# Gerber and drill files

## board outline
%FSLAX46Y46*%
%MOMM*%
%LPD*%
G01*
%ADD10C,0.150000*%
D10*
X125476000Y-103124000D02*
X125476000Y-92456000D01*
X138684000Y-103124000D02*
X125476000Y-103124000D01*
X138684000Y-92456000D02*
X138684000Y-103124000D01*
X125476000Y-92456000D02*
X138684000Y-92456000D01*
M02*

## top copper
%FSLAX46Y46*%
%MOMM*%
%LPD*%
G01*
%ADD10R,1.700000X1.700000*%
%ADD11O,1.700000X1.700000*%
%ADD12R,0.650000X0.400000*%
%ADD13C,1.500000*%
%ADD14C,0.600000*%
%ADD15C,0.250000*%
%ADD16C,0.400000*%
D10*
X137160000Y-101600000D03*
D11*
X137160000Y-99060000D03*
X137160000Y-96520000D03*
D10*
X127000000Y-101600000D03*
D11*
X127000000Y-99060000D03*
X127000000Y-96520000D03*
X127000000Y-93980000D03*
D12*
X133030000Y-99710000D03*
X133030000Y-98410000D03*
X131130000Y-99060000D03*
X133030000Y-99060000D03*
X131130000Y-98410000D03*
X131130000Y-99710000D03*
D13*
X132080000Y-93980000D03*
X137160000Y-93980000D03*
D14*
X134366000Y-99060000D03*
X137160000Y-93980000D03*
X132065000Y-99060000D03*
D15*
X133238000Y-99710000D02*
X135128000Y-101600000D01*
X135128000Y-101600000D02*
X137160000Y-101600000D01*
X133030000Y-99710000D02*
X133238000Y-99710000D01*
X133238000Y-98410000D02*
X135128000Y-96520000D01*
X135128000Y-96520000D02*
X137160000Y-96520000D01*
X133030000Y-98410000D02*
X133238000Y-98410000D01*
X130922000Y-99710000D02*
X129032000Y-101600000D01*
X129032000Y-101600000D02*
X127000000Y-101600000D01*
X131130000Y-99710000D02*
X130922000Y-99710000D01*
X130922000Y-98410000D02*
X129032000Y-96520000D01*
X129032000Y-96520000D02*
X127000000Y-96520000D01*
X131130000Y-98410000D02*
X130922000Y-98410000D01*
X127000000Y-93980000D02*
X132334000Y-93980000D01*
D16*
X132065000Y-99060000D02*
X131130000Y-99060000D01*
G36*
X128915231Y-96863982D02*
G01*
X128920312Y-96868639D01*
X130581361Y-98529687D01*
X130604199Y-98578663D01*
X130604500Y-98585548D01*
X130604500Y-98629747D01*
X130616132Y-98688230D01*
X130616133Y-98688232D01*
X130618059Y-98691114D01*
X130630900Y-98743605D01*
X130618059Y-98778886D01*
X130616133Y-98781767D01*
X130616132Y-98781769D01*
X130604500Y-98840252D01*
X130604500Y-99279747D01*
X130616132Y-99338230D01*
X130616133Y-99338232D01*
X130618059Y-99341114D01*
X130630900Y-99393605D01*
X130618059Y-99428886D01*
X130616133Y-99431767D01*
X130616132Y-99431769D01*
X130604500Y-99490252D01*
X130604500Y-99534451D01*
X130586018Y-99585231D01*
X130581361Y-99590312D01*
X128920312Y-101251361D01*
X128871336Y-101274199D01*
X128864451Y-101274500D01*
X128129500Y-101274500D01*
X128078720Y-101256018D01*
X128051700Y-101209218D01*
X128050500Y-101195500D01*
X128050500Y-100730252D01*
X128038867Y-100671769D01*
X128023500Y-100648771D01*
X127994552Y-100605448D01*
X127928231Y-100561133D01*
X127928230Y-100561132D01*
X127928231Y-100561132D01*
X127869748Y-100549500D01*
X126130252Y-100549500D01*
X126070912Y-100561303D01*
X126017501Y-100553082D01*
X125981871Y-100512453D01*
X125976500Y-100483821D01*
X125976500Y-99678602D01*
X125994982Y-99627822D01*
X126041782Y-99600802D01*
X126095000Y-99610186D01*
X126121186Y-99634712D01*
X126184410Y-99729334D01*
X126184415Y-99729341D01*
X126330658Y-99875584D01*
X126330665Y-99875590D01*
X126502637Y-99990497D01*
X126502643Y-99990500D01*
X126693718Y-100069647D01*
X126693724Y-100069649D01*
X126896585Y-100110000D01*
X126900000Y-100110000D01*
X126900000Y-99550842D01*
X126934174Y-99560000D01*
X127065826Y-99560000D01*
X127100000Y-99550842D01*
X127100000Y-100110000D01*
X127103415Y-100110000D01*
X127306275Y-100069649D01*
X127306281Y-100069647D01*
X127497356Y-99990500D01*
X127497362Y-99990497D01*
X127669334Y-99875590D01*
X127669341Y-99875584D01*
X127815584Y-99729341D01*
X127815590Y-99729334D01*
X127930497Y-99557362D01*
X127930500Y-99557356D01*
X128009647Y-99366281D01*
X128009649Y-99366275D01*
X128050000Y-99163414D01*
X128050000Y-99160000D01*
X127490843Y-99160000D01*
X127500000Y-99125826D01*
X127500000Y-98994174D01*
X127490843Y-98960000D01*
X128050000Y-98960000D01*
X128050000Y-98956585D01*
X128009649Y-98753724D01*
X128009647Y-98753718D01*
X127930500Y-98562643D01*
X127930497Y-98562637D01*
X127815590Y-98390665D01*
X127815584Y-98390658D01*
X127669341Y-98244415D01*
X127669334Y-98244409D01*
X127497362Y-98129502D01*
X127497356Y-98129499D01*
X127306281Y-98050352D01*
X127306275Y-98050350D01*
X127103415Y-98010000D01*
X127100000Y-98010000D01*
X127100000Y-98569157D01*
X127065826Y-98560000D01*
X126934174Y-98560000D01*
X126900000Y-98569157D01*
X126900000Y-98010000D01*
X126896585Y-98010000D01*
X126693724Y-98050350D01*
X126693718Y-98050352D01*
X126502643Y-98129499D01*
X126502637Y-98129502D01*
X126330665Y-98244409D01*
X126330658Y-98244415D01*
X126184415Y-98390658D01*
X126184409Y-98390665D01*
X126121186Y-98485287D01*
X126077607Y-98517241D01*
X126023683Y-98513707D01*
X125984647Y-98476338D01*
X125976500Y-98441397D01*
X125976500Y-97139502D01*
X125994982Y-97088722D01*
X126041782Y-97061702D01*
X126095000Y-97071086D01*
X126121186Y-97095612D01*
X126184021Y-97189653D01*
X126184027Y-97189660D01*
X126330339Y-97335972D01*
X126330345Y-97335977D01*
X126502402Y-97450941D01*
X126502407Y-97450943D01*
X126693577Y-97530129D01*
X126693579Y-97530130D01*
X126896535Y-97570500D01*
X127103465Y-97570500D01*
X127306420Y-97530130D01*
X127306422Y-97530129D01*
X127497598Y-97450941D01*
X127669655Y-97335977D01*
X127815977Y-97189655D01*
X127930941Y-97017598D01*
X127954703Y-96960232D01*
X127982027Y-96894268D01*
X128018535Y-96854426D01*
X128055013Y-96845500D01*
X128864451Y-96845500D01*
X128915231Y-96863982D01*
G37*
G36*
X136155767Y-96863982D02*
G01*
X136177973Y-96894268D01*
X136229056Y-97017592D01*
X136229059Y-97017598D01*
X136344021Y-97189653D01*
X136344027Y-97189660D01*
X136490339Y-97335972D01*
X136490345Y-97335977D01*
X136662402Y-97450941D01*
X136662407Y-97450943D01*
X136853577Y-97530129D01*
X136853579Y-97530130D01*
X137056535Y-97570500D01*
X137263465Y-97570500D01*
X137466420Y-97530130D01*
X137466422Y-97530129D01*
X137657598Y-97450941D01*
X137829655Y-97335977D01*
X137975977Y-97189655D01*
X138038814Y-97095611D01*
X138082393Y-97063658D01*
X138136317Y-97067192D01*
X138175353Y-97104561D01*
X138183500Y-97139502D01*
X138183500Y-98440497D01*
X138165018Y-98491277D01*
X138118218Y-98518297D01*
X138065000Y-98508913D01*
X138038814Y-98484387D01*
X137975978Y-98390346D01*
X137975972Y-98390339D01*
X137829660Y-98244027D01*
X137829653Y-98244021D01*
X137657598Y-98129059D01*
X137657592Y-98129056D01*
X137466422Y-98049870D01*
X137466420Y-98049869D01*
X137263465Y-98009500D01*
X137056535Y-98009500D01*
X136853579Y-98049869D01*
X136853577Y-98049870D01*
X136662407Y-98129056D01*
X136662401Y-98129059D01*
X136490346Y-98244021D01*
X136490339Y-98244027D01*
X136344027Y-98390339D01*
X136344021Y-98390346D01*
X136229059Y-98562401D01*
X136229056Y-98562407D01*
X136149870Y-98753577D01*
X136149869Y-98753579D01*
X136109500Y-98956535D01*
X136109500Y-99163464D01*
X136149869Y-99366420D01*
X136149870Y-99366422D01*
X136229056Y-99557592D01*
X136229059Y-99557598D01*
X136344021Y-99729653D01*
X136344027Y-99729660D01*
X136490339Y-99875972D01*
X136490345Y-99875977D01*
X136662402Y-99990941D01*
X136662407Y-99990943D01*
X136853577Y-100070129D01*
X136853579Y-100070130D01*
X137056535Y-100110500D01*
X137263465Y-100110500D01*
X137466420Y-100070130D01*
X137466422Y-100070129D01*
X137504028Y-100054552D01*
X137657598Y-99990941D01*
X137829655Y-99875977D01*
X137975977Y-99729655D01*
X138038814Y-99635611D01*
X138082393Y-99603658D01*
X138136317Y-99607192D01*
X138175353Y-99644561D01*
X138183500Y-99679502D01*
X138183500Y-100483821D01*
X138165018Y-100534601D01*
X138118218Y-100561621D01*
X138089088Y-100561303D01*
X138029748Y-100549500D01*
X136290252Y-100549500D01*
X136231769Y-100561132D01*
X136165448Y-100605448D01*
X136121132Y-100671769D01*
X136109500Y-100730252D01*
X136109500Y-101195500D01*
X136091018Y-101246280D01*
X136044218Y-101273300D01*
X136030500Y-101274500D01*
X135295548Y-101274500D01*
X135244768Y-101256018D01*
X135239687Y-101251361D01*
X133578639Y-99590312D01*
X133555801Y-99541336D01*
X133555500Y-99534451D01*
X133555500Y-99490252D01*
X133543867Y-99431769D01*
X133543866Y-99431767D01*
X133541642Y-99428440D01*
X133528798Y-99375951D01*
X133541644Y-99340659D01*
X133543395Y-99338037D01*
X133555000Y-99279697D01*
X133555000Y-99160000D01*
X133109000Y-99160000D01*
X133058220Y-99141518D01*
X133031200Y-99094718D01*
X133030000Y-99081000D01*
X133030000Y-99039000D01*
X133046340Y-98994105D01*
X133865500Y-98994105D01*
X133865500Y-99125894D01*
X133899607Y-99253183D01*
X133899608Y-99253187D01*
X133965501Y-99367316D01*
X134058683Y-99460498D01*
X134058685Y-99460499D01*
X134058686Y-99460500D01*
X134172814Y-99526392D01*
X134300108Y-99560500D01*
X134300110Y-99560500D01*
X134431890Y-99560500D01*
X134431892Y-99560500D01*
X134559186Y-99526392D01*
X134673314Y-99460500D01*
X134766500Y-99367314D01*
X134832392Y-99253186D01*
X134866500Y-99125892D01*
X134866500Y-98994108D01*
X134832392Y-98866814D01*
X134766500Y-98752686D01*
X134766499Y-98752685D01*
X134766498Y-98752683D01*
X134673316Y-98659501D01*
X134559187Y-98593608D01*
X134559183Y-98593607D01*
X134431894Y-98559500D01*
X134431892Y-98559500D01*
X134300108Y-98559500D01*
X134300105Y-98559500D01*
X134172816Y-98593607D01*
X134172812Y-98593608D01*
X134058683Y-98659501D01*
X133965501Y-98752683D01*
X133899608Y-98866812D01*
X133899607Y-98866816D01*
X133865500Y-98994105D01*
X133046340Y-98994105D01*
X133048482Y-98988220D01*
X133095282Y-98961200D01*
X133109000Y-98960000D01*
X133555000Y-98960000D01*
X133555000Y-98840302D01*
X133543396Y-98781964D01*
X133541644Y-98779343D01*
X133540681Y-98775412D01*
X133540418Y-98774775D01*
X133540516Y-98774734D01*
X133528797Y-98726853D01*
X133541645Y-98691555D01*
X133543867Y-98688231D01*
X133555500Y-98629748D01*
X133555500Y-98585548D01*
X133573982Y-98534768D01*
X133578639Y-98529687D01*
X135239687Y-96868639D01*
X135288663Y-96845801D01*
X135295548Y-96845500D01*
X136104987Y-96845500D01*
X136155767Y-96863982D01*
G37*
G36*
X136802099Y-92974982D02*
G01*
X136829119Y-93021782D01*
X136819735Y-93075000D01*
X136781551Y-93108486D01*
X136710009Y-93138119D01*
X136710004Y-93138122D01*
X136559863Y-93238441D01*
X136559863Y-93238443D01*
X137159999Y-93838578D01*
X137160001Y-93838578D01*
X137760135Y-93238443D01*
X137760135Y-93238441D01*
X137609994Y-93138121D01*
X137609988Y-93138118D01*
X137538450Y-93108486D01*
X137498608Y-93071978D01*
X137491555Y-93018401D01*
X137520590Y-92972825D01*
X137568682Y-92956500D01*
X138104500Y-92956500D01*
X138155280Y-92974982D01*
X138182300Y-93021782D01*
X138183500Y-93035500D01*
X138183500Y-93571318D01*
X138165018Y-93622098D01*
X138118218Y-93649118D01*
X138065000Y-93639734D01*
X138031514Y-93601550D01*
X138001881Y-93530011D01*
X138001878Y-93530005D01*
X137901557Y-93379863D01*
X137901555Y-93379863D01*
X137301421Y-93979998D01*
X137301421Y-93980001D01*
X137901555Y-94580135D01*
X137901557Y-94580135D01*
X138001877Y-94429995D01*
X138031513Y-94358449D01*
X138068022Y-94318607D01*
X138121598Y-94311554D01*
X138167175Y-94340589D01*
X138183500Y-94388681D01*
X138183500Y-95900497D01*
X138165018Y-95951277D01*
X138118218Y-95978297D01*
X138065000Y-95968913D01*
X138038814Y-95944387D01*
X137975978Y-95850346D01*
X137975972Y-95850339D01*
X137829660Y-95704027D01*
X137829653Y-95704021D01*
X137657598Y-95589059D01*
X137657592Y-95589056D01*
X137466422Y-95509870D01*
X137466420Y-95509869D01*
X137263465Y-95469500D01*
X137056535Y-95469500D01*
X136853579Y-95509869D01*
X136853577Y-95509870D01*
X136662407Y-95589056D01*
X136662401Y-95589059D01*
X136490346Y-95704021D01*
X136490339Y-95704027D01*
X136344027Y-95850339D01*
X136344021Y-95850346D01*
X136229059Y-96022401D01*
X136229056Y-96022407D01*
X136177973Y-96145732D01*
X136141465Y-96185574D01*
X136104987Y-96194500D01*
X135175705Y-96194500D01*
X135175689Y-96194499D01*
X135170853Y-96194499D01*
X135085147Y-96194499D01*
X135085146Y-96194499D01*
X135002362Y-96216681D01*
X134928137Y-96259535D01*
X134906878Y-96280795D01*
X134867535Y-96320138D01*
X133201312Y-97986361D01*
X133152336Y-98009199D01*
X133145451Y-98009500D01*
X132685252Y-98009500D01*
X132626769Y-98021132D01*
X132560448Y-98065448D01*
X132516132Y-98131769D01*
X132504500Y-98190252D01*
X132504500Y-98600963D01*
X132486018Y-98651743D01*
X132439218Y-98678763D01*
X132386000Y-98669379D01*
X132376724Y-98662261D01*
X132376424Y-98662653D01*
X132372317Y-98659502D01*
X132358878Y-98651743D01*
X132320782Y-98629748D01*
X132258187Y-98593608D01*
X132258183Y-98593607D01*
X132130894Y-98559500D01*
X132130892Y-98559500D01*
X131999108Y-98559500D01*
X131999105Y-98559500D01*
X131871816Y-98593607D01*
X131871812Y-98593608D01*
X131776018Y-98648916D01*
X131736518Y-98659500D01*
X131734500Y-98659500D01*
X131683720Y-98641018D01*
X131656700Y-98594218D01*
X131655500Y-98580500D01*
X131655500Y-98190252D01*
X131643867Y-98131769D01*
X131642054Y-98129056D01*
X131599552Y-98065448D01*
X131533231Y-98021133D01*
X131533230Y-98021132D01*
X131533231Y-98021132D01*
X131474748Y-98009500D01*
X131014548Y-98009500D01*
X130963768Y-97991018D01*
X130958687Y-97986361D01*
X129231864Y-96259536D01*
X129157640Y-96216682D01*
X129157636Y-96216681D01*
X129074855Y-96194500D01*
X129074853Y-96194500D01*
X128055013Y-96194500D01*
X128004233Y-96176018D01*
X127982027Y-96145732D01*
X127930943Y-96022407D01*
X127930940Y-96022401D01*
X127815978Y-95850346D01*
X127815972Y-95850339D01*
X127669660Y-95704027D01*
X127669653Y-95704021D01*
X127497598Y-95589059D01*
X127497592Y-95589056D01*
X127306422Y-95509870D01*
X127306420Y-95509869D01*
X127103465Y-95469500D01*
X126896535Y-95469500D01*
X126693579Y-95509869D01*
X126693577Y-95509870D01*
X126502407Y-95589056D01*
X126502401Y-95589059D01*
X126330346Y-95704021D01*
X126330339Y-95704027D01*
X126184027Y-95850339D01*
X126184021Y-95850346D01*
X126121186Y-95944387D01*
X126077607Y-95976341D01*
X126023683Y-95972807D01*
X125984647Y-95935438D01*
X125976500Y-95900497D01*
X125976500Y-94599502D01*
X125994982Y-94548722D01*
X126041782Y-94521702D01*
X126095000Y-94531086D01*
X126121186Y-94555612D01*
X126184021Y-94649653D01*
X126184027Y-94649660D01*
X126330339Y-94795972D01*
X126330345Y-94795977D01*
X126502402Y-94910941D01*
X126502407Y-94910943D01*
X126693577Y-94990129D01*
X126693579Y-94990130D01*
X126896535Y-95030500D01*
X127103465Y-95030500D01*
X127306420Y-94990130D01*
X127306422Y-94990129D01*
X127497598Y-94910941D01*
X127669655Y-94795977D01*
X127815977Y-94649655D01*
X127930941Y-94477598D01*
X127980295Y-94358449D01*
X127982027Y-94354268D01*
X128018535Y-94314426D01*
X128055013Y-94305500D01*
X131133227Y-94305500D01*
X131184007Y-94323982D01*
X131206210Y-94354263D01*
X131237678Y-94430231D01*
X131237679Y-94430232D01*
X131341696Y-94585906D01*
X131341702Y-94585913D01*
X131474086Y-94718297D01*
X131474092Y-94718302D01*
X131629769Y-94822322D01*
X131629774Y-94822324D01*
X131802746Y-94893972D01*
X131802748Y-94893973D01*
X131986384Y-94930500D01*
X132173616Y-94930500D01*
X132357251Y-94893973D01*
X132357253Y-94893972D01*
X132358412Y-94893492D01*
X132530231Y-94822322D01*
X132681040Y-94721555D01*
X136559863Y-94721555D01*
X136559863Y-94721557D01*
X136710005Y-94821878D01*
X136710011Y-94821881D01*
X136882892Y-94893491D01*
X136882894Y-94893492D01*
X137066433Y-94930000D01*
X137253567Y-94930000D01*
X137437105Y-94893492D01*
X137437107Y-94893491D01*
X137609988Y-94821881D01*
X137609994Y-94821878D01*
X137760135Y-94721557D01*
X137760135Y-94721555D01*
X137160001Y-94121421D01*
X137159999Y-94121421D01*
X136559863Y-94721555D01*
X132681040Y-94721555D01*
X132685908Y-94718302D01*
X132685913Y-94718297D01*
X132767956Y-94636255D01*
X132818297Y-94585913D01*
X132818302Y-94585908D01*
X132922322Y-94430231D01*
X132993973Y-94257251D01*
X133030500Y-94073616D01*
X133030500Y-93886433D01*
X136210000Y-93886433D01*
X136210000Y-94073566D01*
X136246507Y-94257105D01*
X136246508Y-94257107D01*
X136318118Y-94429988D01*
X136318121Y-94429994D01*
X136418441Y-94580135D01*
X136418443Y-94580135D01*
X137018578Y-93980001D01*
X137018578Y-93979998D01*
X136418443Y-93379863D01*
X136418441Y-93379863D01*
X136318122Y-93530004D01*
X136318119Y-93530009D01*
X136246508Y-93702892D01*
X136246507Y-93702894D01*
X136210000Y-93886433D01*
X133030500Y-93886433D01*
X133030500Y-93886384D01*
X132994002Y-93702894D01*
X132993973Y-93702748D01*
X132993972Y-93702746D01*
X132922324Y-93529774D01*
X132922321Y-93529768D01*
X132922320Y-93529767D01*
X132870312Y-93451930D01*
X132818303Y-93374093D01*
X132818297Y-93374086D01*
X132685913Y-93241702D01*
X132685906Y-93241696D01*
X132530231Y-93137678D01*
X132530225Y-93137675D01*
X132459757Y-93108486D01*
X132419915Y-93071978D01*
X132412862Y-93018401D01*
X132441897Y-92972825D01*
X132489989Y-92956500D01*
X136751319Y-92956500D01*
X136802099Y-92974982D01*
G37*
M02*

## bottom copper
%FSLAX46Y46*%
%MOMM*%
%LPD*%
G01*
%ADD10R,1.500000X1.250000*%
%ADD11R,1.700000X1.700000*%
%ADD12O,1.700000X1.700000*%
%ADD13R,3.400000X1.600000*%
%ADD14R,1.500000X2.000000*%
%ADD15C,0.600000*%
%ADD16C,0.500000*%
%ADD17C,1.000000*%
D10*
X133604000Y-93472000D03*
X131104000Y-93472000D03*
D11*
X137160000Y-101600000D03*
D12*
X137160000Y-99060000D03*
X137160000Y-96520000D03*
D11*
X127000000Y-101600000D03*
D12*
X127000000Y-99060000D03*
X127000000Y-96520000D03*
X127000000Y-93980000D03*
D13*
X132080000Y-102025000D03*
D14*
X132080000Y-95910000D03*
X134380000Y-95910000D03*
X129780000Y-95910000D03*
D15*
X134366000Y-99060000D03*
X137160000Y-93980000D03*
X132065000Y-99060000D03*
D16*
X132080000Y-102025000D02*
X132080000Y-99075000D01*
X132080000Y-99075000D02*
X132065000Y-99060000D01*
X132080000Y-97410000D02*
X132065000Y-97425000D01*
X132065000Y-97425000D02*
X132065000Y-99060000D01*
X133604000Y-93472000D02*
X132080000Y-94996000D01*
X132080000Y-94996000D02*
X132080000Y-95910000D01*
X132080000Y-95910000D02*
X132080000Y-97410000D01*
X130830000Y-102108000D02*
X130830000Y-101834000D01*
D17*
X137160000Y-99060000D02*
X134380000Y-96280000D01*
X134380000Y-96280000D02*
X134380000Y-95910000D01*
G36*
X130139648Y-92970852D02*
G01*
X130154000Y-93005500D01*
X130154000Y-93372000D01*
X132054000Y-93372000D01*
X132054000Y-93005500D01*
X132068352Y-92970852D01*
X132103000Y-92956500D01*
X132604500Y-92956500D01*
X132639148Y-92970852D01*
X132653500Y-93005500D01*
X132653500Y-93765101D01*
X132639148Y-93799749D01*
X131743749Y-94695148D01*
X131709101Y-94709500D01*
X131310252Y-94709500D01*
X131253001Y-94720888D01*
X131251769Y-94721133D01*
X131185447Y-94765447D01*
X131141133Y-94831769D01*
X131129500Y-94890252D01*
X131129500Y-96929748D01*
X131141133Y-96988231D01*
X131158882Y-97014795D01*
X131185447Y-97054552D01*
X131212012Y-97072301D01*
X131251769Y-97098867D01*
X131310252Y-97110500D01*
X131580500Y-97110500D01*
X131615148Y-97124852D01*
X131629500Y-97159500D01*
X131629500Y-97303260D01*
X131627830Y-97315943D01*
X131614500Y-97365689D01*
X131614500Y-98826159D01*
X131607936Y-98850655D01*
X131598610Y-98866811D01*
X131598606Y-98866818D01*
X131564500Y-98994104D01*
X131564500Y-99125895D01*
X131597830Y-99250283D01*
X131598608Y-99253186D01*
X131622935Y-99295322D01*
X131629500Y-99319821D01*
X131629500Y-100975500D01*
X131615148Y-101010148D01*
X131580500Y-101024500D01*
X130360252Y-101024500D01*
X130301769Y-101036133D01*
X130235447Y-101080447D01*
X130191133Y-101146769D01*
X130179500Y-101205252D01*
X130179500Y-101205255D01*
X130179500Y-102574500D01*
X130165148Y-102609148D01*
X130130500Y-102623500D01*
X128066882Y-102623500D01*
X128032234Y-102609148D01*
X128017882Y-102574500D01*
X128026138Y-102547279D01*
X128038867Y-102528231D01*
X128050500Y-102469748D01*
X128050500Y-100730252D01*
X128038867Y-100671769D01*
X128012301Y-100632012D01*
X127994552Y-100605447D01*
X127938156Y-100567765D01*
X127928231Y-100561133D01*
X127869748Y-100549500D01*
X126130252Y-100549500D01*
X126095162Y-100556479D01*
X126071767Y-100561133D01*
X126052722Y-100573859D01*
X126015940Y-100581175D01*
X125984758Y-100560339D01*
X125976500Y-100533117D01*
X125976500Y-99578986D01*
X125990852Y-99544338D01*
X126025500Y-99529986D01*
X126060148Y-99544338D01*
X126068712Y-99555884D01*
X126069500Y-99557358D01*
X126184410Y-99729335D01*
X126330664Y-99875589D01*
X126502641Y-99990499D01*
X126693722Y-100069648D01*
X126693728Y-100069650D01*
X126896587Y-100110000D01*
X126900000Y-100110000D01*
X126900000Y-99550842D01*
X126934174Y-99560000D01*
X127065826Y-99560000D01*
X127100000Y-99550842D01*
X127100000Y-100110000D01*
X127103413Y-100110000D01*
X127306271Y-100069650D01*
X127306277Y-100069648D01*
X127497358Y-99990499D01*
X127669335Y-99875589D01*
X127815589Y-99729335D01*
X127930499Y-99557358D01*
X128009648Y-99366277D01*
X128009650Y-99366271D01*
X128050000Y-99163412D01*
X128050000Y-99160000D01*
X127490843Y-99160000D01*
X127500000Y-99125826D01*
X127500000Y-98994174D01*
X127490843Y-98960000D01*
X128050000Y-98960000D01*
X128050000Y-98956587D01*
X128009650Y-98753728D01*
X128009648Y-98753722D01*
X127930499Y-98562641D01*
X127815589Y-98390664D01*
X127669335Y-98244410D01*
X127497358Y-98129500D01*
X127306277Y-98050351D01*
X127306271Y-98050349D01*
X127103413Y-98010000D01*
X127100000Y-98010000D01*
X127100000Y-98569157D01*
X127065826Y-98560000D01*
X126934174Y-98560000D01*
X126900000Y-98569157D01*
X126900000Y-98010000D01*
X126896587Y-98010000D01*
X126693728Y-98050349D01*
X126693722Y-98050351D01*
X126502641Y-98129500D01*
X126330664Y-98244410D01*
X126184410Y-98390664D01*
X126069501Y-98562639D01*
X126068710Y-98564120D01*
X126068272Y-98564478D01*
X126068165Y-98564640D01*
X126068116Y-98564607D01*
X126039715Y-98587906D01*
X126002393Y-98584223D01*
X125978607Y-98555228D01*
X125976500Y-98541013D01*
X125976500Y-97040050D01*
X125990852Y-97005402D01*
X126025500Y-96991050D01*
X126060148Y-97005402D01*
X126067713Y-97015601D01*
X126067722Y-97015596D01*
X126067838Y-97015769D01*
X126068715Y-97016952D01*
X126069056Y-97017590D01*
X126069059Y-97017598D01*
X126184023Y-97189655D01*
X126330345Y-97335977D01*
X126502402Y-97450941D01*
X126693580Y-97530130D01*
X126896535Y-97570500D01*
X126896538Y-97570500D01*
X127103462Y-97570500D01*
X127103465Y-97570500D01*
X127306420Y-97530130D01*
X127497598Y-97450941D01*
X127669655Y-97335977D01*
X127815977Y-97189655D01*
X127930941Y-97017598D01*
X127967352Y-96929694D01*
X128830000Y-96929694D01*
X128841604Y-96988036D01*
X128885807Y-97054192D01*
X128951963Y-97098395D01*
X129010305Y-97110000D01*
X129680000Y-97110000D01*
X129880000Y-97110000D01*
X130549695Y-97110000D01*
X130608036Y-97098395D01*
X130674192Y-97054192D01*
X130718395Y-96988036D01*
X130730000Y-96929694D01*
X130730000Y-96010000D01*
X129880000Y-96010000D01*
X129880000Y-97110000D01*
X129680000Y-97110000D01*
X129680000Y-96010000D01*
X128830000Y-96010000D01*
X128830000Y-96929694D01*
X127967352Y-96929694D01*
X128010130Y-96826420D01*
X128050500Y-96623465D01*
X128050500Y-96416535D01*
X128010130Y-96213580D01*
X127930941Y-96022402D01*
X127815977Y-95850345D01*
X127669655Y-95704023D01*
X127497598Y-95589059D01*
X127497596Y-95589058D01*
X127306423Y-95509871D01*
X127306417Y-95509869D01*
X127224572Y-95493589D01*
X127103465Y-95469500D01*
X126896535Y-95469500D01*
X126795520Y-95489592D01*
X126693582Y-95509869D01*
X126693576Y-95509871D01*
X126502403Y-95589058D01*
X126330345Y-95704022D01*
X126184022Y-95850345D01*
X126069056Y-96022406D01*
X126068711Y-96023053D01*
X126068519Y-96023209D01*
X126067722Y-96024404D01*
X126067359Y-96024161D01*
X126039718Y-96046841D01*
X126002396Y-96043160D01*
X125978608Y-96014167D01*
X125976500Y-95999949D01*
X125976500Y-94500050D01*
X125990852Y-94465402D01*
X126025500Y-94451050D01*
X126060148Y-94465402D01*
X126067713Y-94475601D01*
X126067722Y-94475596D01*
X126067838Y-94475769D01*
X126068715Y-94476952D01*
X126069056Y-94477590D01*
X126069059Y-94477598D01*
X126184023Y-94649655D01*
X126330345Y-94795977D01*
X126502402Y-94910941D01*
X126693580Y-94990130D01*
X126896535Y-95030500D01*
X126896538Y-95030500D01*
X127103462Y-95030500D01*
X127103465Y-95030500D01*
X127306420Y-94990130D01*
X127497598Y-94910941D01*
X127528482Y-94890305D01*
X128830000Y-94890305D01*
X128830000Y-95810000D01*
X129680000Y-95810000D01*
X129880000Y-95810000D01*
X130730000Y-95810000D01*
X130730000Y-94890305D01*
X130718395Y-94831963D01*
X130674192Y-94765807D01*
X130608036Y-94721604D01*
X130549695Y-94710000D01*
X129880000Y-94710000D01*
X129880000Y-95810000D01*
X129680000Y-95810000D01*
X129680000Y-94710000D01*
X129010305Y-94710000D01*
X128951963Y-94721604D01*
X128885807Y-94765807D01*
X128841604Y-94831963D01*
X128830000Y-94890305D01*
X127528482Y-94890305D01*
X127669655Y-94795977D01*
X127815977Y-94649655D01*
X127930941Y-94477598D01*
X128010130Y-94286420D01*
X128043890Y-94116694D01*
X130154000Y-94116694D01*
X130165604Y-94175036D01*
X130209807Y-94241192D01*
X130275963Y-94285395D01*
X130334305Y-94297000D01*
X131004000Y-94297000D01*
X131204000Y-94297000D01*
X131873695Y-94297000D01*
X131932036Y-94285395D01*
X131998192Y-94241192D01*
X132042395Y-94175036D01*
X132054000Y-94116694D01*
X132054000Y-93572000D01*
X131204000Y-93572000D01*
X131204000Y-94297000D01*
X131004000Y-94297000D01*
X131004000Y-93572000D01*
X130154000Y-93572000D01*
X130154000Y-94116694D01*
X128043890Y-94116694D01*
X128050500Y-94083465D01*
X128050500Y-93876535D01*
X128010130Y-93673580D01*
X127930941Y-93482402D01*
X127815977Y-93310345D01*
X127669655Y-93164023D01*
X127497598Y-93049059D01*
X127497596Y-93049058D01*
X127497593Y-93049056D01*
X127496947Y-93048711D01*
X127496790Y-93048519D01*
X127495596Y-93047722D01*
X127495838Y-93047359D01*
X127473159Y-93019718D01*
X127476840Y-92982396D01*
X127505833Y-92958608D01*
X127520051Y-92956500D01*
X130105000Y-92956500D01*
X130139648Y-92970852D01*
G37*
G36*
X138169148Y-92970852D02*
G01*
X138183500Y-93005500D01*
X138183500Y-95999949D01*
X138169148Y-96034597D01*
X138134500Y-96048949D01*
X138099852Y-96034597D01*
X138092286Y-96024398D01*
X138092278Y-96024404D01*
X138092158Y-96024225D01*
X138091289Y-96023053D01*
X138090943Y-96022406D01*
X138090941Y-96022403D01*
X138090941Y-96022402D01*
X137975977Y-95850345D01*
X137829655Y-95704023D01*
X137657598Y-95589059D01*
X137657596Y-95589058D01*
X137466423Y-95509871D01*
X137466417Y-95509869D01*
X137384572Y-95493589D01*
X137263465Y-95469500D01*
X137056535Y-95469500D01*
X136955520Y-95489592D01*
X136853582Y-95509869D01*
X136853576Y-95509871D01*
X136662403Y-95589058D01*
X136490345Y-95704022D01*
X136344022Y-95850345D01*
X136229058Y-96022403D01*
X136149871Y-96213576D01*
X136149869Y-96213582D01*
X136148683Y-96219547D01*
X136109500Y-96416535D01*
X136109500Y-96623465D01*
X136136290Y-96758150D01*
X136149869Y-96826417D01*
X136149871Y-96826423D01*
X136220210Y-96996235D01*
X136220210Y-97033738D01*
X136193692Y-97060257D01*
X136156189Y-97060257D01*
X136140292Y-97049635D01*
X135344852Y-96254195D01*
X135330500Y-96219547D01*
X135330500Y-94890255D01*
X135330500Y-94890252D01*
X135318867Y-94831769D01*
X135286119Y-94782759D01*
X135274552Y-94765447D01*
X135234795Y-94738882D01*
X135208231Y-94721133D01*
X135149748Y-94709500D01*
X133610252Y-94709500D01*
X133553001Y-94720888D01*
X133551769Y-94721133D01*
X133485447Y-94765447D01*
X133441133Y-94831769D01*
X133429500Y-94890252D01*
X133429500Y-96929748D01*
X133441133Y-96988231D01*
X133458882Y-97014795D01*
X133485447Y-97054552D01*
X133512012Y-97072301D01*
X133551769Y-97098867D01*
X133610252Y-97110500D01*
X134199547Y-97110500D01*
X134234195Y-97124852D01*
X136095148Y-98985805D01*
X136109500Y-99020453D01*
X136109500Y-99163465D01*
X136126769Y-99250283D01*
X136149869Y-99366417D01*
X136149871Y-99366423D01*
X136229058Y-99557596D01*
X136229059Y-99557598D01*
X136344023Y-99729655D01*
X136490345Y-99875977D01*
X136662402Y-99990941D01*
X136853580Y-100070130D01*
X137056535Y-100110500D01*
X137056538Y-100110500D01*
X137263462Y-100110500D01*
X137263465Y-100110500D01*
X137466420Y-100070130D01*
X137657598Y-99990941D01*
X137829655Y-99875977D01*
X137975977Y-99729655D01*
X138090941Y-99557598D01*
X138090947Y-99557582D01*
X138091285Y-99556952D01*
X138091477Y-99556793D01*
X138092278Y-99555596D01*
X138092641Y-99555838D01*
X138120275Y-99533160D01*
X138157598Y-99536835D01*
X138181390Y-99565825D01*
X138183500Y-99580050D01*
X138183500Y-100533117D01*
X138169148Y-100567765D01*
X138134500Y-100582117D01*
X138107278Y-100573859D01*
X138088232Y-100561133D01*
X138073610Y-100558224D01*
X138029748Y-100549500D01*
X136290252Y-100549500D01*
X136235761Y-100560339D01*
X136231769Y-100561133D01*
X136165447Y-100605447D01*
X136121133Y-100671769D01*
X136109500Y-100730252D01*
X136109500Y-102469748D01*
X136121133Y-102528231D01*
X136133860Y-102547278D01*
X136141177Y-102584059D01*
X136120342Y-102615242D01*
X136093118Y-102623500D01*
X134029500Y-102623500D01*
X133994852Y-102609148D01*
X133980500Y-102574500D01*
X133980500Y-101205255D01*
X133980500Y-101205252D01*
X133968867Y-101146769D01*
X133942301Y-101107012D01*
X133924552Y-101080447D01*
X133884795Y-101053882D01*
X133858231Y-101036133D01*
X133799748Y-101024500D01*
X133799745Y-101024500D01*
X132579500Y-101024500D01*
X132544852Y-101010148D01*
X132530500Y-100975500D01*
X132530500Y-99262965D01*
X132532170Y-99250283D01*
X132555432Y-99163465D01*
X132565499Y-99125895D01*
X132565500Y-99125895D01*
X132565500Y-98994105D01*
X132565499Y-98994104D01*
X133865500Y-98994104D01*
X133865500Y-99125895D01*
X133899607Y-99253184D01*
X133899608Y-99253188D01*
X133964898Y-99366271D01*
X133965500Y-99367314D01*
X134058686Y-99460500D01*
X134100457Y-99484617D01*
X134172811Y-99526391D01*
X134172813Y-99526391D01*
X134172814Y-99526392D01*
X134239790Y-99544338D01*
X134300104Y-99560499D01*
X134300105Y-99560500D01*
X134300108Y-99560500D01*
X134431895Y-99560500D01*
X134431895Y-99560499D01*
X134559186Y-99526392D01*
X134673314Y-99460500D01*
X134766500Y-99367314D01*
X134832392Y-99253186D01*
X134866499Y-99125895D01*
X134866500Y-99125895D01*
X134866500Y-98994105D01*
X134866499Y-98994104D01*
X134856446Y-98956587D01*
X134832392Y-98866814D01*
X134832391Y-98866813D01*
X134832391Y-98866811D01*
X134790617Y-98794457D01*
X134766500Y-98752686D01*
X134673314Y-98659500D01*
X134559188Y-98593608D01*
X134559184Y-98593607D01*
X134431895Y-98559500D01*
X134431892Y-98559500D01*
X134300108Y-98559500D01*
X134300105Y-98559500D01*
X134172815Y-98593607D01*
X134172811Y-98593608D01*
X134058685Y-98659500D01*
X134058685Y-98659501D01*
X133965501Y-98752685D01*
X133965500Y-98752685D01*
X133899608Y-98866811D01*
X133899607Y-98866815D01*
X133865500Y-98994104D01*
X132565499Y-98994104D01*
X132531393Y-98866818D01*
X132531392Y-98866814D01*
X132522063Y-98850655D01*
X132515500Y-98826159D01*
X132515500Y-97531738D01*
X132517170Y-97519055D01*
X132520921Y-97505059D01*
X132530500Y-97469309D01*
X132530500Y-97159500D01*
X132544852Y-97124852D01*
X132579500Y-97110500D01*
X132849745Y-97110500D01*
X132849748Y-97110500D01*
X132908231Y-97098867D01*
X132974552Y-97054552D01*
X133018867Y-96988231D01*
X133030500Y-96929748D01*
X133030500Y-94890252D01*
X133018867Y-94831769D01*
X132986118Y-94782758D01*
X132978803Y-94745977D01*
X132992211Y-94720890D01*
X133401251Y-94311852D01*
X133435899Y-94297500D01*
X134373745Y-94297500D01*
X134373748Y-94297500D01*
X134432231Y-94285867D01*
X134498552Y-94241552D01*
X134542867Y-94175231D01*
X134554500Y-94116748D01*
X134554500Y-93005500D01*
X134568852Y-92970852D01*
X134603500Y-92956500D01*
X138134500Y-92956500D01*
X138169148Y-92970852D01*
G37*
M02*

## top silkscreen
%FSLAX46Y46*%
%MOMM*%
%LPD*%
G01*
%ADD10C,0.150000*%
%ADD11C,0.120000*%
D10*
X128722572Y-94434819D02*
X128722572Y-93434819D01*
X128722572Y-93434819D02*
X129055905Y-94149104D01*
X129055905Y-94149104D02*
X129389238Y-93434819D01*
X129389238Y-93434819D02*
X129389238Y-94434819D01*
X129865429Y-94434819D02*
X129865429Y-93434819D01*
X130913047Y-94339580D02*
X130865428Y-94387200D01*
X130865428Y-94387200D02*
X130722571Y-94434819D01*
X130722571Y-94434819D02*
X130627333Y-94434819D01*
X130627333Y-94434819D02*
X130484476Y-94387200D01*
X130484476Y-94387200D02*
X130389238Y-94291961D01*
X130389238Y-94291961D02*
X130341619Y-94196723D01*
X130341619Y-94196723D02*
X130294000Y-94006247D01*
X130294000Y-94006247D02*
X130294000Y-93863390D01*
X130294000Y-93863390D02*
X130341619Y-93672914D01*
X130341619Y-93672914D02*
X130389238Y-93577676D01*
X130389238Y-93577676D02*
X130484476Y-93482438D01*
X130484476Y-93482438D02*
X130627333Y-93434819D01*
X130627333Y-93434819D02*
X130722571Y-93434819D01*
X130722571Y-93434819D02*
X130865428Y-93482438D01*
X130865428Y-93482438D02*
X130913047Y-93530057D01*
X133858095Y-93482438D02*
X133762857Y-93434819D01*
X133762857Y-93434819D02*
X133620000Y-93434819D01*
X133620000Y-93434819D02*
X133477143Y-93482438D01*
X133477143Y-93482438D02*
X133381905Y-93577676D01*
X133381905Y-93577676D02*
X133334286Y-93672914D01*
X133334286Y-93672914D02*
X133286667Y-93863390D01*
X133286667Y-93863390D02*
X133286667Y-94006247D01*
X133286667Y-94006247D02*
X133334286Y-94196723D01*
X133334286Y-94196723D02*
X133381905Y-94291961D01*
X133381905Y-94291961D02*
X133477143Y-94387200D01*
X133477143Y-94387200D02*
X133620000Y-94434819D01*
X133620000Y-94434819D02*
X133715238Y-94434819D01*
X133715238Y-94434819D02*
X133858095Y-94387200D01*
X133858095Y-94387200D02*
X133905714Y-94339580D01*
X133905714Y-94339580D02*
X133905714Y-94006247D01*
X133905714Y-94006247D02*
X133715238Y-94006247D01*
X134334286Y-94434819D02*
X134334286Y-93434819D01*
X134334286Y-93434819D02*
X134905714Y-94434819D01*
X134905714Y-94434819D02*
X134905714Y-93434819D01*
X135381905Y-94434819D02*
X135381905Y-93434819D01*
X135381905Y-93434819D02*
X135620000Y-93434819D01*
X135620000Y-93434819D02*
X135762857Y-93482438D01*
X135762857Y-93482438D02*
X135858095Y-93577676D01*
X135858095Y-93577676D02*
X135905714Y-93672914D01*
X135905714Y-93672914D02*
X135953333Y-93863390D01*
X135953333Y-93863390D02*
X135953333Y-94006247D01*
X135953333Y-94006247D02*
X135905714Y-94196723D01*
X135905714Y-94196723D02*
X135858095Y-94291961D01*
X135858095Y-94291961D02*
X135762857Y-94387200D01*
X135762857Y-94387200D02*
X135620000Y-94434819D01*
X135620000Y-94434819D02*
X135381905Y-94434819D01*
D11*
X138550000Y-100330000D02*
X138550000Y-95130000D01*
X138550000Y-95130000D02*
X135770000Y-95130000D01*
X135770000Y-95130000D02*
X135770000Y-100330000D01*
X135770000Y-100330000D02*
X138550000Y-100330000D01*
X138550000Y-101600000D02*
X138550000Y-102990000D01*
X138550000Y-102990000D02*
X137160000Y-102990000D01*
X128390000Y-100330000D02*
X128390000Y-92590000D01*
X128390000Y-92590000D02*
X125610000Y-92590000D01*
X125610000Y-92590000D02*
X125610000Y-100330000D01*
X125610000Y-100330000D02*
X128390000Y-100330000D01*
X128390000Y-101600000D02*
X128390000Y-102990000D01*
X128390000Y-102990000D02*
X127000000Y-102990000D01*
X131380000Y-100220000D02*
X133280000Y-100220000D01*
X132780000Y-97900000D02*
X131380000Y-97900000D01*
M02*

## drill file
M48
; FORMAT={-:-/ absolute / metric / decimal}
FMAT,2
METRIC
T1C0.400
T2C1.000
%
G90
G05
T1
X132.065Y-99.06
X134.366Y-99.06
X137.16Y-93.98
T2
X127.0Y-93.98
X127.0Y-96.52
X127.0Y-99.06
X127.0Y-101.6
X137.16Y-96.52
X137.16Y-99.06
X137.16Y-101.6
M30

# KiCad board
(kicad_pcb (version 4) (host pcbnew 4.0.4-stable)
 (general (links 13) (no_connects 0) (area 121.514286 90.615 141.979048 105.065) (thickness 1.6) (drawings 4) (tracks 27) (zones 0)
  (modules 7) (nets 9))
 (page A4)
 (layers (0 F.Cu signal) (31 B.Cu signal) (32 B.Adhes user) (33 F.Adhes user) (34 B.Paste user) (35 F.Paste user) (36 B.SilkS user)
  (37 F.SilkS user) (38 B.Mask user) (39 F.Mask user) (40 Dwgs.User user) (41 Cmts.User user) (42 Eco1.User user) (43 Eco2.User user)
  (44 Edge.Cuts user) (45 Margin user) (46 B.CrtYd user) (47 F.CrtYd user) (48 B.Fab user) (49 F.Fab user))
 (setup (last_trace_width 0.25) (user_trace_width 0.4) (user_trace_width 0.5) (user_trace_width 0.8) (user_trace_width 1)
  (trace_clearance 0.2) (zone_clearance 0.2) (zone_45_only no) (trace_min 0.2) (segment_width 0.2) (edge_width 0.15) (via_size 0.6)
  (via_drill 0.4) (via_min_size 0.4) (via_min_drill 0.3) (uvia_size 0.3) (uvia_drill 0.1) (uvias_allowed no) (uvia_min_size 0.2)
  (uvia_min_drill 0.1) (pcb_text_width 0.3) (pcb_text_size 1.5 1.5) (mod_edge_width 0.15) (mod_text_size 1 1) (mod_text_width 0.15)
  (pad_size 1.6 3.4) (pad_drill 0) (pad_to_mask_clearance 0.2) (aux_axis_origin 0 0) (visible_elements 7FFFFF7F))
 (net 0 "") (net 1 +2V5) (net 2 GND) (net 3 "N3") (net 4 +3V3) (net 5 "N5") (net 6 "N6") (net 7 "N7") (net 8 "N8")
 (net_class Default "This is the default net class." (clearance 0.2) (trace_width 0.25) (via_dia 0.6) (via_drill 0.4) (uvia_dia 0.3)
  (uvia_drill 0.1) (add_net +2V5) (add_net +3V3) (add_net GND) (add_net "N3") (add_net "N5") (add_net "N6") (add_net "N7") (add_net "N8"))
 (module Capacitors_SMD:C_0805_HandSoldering (layer B.Cu) (at 132.354 93.472 180)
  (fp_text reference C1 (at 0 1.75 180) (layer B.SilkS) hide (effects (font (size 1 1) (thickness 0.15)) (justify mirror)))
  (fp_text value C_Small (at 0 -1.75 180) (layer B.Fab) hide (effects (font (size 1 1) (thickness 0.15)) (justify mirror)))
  (pad 1 smd rect (at -1.25 0 180) (size 1.5 1.25) (layers B.Cu B.Paste B.Mask) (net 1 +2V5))
  (pad 2 smd rect (at 1.25 0 180) (size 1.5 1.25) (layers B.Cu B.Paste B.Mask) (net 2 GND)))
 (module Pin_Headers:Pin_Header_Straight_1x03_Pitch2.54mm (layer F.Cu) (at 137.16 101.6 180)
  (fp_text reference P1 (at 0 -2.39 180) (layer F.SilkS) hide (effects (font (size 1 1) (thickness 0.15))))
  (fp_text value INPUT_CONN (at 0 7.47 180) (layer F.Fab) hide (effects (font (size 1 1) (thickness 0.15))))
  (fp_line (start -1.39 1.27) (end -1.39 6.47) (layer F.SilkS) (width 0.12))
  (fp_line (start -1.39 6.47) (end 1.39 6.47) (layer F.SilkS) (width 0.12))
  (fp_line (start 1.39 6.47) (end 1.39 1.27) (layer F.SilkS) (width 0.12))
  (fp_line (start 1.39 1.27) (end -1.39 1.27) (layer F.SilkS) (width 0.12))
  (fp_line (start -1.39 0) (end -1.39 -1.39) (layer F.SilkS) (width 0.12))
  (fp_line (start -1.39 -1.39) (end 0 -1.39) (layer F.SilkS) (width 0.12))
  (pad 1 thru_hole rect (at 0 0 180) (size 1.7 1.7) (drill 1) (layers *.Cu *.Mask) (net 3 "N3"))
  (pad 2 thru_hole oval (at 0 2.54 180) (size 1.7 1.7) (drill 1) (layers *.Cu *.Mask) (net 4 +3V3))
  (pad 3 thru_hole oval (at 0 5.08 180) (size 1.7 1.7) (drill 1) (layers *.Cu *.Mask) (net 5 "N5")))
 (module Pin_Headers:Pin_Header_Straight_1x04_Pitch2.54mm (layer F.Cu) (at 127 101.6 180)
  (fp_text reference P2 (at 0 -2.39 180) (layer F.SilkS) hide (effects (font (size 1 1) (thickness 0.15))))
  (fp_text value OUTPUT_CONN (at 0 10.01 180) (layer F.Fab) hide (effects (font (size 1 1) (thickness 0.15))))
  (fp_line (start -1.39 1.27) (end -1.39 9.01) (layer F.SilkS) (width 0.12))
  (fp_line (start -1.39 9.01) (end 1.39 9.01) (layer F.SilkS) (width 0.12))
  (fp_line (start 1.39 9.01) (end 1.39 1.27) (layer F.SilkS) (width 0.12))
  (fp_line (start 1.39 1.27) (end -1.39 1.27) (layer F.SilkS) (width 0.12))
  (fp_line (start -1.39 0) (end -1.39 -1.39) (layer F.SilkS) (width 0.12))
  (fp_line (start -1.39 -1.39) (end 0 -1.39) (layer F.SilkS) (width 0.12))
  (pad 1 thru_hole rect (at 0 0 180) (size 1.7 1.7) (drill 1) (layers *.Cu *.Mask) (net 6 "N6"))
  (pad 2 thru_hole oval (at 0 2.54 180) (size 1.7 1.7) (drill 1) (layers *.Cu *.Mask) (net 2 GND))
  (pad 3 thru_hole oval (at 0 5.08 180) (size 1.7 1.7) (drill 1) (layers *.Cu *.Mask) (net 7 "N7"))
  (pad 4 thru_hole oval (at 0 7.62 180) (size 1.7 1.7) (drill 1) (layers *.Cu *.Mask) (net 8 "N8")))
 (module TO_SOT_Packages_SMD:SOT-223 (layer B.Cu) (at 132.08 99.06 270)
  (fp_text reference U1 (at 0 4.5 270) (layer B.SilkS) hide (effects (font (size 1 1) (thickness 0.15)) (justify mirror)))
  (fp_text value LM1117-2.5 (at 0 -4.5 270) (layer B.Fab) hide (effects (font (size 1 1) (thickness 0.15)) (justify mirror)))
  (pad 4 smd rect (at 2.965 0 270) (size 1.6 3.4) (layers B.Cu B.Paste B.Mask) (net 1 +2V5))
  (pad 2 smd rect (at -3.15 0 270) (size 2 1.5) (layers B.Cu B.Paste B.Mask) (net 1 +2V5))
  (pad 3 smd rect (at -3.15 -2.3 270) (size 2 1.5) (layers B.Cu B.Paste B.Mask) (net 4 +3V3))
  (pad 1 smd rect (at -3.15 2.3 270) (size 2 1.5) (layers B.Cu B.Paste B.Mask) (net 2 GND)))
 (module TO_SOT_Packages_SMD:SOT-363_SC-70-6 (layer F.Cu) (at 132.08 99.06 180)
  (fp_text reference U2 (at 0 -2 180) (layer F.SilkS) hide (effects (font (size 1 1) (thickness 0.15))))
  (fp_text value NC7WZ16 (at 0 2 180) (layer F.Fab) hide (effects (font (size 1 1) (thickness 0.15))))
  (fp_line (start 0.7 -1.16) (end -1.2 -1.16) (layer F.SilkS) (width 0.12))
  (fp_line (start -0.7 1.16) (end 0.7 1.16) (layer F.SilkS) (width 0.12))
  (pad 1 smd rect (at -0.95 -0.65 180) (size 0.65 0.4) (layers F.Cu F.Paste F.Mask) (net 3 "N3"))
  (pad 3 smd rect (at -0.95 0.65 180) (size 0.65 0.4) (layers F.Cu F.Paste F.Mask) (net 5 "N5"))
  (pad 5 smd rect (at 0.95 0 180) (size 0.65 0.4) (layers F.Cu F.Paste F.Mask) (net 1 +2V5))
  (pad 2 smd rect (at -0.95 0 180) (size 0.65 0.4) (layers F.Cu F.Paste F.Mask) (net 2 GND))
  (pad 4 smd rect (at 0.95 0.65 180) (size 0.65 0.4) (layers F.Cu F.Paste F.Mask) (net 7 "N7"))
  (pad 6 smd rect (at 0.95 -0.65 180) (size 0.65 0.4) (layers F.Cu F.Paste F.Mask) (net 6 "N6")))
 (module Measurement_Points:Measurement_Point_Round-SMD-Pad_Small (layer F.Cu) (at 132.08 93.98)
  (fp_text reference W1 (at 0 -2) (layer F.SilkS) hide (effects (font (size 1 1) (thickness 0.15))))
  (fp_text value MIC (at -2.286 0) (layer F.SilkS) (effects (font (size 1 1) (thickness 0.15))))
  (pad 1 smd circle (at 0 0) (size 1.5 1.5) (layers F.Cu F.Mask) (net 8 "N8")))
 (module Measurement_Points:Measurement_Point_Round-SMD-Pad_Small (layer F.Cu) (at 137.16 93.98)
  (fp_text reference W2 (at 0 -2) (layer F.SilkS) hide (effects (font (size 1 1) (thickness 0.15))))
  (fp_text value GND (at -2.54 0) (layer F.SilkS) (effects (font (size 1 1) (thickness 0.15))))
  (pad 1 smd circle (at 0 0) (size 1.5 1.5) (layers F.Cu F.Mask) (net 2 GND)))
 (gr_line (start 125.476 103.124) (end 125.476 92.456) (layer Edge.Cuts) (width 0.15))
 (gr_line (start 138.684 103.124) (end 125.476 103.124) (layer Edge.Cuts) (width 0.15))
 (gr_line (start 138.684 92.456) (end 138.684 103.124) (layer Edge.Cuts) (width 0.15))
 (gr_line (start 125.476 92.456) (end 138.684 92.456) (layer Edge.Cuts) (width 0.15))
 (via (at 134.366 99.06) (size 0.6) (drill 0.4) (layers F.Cu B.Cu) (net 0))
 (via (at 137.16 93.98) (size 0.6) (drill 0.4) (layers F.Cu B.Cu) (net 2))
 (segment (start 133.238 99.71) (end 135.128 101.6) (width 0.25) (layer F.Cu) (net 3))
 (segment (start 135.128 101.6) (end 137.16 101.6) (width 0.25) (layer F.Cu) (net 3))
 (segment (start 133.03 99.71) (end 133.238 99.71) (width 0.25) (layer F.Cu) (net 3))
 (segment (start 133.238 98.41) (end 135.128 96.52) (width 0.25) (layer F.Cu) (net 5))
 (segment (start 135.128 96.52) (end 137.16 96.52) (width 0.25) (layer F.Cu) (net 5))
 (segment (start 133.03 98.41) (end 133.238 98.41) (width 0.25) (layer F.Cu) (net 5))
 (segment (start 130.922 99.71) (end 129.032 101.6) (width 0.25) (layer F.Cu) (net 6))
 (segment (start 129.032 101.6) (end 127 101.6) (width 0.25) (layer F.Cu) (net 6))
 (segment (start 131.13 99.71) (end 130.922 99.71) (width 0.25) (layer F.Cu) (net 6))
 (segment (start 130.922 98.41) (end 129.032 96.52) (width 0.25) (layer F.Cu) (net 7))
 (segment (start 129.032 96.52) (end 127 96.52) (width 0.25) (layer F.Cu) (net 7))
 (segment (start 131.13 98.41) (end 130.922 98.41) (width 0.25) (layer F.Cu) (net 7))
 (segment (start 127 93.98) (end 132.334 93.98) (width 0.25) (layer F.Cu) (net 8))
 (segment (start 132.08 102.025) (end 132.08 99.075) (width 0.5) (layer B.Cu) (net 1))
 (segment (start 132.08 99.075) (end 132.065 99.06) (width 0.5) (layer B.Cu) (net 1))
 (segment (start 132.065 99.06) (end 131.13 99.06) (width 0.4) (layer F.Cu) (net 1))
 (segment (start 132.08 97.41) (end 132.065 97.425) (width 0.5) (layer B.Cu) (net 1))
 (segment (start 132.065 97.425) (end 132.065 99.06) (width 0.5) (layer B.Cu) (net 1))
 (segment (start 133.604 93.472) (end 132.08 94.996) (width 0.5) (layer B.Cu) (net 1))
 (segment (start 132.08 94.996) (end 132.08 95.91) (width 0.5) (layer B.Cu) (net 1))
 (via (at 132.065 99.06) (size 0.6) (drill 0.4) (layers F.Cu B.Cu) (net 1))
 (segment (start 132.08 95.91) (end 132.08 97.41) (width 0.5) (layer B.Cu) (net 1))
 (segment (start 130.83 102.108) (end 130.83 101.834) (width 0.5) (layer B.Cu) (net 1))
 (segment (start 137.16 99.06) (end 134.38 96.28) (width 1) (layer B.Cu) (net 4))
 (segment (start 134.38 96.28) (end 134.38 95.91) (width 1) (layer B.Cu) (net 4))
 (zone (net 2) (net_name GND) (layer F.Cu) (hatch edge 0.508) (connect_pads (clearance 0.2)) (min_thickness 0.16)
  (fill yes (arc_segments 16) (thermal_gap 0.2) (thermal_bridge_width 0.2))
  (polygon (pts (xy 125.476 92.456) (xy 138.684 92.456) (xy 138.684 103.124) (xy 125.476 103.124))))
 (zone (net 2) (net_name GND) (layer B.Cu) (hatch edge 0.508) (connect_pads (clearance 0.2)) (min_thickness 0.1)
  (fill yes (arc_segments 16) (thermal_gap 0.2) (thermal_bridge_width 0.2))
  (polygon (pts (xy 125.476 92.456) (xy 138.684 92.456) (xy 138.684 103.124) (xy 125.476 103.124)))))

